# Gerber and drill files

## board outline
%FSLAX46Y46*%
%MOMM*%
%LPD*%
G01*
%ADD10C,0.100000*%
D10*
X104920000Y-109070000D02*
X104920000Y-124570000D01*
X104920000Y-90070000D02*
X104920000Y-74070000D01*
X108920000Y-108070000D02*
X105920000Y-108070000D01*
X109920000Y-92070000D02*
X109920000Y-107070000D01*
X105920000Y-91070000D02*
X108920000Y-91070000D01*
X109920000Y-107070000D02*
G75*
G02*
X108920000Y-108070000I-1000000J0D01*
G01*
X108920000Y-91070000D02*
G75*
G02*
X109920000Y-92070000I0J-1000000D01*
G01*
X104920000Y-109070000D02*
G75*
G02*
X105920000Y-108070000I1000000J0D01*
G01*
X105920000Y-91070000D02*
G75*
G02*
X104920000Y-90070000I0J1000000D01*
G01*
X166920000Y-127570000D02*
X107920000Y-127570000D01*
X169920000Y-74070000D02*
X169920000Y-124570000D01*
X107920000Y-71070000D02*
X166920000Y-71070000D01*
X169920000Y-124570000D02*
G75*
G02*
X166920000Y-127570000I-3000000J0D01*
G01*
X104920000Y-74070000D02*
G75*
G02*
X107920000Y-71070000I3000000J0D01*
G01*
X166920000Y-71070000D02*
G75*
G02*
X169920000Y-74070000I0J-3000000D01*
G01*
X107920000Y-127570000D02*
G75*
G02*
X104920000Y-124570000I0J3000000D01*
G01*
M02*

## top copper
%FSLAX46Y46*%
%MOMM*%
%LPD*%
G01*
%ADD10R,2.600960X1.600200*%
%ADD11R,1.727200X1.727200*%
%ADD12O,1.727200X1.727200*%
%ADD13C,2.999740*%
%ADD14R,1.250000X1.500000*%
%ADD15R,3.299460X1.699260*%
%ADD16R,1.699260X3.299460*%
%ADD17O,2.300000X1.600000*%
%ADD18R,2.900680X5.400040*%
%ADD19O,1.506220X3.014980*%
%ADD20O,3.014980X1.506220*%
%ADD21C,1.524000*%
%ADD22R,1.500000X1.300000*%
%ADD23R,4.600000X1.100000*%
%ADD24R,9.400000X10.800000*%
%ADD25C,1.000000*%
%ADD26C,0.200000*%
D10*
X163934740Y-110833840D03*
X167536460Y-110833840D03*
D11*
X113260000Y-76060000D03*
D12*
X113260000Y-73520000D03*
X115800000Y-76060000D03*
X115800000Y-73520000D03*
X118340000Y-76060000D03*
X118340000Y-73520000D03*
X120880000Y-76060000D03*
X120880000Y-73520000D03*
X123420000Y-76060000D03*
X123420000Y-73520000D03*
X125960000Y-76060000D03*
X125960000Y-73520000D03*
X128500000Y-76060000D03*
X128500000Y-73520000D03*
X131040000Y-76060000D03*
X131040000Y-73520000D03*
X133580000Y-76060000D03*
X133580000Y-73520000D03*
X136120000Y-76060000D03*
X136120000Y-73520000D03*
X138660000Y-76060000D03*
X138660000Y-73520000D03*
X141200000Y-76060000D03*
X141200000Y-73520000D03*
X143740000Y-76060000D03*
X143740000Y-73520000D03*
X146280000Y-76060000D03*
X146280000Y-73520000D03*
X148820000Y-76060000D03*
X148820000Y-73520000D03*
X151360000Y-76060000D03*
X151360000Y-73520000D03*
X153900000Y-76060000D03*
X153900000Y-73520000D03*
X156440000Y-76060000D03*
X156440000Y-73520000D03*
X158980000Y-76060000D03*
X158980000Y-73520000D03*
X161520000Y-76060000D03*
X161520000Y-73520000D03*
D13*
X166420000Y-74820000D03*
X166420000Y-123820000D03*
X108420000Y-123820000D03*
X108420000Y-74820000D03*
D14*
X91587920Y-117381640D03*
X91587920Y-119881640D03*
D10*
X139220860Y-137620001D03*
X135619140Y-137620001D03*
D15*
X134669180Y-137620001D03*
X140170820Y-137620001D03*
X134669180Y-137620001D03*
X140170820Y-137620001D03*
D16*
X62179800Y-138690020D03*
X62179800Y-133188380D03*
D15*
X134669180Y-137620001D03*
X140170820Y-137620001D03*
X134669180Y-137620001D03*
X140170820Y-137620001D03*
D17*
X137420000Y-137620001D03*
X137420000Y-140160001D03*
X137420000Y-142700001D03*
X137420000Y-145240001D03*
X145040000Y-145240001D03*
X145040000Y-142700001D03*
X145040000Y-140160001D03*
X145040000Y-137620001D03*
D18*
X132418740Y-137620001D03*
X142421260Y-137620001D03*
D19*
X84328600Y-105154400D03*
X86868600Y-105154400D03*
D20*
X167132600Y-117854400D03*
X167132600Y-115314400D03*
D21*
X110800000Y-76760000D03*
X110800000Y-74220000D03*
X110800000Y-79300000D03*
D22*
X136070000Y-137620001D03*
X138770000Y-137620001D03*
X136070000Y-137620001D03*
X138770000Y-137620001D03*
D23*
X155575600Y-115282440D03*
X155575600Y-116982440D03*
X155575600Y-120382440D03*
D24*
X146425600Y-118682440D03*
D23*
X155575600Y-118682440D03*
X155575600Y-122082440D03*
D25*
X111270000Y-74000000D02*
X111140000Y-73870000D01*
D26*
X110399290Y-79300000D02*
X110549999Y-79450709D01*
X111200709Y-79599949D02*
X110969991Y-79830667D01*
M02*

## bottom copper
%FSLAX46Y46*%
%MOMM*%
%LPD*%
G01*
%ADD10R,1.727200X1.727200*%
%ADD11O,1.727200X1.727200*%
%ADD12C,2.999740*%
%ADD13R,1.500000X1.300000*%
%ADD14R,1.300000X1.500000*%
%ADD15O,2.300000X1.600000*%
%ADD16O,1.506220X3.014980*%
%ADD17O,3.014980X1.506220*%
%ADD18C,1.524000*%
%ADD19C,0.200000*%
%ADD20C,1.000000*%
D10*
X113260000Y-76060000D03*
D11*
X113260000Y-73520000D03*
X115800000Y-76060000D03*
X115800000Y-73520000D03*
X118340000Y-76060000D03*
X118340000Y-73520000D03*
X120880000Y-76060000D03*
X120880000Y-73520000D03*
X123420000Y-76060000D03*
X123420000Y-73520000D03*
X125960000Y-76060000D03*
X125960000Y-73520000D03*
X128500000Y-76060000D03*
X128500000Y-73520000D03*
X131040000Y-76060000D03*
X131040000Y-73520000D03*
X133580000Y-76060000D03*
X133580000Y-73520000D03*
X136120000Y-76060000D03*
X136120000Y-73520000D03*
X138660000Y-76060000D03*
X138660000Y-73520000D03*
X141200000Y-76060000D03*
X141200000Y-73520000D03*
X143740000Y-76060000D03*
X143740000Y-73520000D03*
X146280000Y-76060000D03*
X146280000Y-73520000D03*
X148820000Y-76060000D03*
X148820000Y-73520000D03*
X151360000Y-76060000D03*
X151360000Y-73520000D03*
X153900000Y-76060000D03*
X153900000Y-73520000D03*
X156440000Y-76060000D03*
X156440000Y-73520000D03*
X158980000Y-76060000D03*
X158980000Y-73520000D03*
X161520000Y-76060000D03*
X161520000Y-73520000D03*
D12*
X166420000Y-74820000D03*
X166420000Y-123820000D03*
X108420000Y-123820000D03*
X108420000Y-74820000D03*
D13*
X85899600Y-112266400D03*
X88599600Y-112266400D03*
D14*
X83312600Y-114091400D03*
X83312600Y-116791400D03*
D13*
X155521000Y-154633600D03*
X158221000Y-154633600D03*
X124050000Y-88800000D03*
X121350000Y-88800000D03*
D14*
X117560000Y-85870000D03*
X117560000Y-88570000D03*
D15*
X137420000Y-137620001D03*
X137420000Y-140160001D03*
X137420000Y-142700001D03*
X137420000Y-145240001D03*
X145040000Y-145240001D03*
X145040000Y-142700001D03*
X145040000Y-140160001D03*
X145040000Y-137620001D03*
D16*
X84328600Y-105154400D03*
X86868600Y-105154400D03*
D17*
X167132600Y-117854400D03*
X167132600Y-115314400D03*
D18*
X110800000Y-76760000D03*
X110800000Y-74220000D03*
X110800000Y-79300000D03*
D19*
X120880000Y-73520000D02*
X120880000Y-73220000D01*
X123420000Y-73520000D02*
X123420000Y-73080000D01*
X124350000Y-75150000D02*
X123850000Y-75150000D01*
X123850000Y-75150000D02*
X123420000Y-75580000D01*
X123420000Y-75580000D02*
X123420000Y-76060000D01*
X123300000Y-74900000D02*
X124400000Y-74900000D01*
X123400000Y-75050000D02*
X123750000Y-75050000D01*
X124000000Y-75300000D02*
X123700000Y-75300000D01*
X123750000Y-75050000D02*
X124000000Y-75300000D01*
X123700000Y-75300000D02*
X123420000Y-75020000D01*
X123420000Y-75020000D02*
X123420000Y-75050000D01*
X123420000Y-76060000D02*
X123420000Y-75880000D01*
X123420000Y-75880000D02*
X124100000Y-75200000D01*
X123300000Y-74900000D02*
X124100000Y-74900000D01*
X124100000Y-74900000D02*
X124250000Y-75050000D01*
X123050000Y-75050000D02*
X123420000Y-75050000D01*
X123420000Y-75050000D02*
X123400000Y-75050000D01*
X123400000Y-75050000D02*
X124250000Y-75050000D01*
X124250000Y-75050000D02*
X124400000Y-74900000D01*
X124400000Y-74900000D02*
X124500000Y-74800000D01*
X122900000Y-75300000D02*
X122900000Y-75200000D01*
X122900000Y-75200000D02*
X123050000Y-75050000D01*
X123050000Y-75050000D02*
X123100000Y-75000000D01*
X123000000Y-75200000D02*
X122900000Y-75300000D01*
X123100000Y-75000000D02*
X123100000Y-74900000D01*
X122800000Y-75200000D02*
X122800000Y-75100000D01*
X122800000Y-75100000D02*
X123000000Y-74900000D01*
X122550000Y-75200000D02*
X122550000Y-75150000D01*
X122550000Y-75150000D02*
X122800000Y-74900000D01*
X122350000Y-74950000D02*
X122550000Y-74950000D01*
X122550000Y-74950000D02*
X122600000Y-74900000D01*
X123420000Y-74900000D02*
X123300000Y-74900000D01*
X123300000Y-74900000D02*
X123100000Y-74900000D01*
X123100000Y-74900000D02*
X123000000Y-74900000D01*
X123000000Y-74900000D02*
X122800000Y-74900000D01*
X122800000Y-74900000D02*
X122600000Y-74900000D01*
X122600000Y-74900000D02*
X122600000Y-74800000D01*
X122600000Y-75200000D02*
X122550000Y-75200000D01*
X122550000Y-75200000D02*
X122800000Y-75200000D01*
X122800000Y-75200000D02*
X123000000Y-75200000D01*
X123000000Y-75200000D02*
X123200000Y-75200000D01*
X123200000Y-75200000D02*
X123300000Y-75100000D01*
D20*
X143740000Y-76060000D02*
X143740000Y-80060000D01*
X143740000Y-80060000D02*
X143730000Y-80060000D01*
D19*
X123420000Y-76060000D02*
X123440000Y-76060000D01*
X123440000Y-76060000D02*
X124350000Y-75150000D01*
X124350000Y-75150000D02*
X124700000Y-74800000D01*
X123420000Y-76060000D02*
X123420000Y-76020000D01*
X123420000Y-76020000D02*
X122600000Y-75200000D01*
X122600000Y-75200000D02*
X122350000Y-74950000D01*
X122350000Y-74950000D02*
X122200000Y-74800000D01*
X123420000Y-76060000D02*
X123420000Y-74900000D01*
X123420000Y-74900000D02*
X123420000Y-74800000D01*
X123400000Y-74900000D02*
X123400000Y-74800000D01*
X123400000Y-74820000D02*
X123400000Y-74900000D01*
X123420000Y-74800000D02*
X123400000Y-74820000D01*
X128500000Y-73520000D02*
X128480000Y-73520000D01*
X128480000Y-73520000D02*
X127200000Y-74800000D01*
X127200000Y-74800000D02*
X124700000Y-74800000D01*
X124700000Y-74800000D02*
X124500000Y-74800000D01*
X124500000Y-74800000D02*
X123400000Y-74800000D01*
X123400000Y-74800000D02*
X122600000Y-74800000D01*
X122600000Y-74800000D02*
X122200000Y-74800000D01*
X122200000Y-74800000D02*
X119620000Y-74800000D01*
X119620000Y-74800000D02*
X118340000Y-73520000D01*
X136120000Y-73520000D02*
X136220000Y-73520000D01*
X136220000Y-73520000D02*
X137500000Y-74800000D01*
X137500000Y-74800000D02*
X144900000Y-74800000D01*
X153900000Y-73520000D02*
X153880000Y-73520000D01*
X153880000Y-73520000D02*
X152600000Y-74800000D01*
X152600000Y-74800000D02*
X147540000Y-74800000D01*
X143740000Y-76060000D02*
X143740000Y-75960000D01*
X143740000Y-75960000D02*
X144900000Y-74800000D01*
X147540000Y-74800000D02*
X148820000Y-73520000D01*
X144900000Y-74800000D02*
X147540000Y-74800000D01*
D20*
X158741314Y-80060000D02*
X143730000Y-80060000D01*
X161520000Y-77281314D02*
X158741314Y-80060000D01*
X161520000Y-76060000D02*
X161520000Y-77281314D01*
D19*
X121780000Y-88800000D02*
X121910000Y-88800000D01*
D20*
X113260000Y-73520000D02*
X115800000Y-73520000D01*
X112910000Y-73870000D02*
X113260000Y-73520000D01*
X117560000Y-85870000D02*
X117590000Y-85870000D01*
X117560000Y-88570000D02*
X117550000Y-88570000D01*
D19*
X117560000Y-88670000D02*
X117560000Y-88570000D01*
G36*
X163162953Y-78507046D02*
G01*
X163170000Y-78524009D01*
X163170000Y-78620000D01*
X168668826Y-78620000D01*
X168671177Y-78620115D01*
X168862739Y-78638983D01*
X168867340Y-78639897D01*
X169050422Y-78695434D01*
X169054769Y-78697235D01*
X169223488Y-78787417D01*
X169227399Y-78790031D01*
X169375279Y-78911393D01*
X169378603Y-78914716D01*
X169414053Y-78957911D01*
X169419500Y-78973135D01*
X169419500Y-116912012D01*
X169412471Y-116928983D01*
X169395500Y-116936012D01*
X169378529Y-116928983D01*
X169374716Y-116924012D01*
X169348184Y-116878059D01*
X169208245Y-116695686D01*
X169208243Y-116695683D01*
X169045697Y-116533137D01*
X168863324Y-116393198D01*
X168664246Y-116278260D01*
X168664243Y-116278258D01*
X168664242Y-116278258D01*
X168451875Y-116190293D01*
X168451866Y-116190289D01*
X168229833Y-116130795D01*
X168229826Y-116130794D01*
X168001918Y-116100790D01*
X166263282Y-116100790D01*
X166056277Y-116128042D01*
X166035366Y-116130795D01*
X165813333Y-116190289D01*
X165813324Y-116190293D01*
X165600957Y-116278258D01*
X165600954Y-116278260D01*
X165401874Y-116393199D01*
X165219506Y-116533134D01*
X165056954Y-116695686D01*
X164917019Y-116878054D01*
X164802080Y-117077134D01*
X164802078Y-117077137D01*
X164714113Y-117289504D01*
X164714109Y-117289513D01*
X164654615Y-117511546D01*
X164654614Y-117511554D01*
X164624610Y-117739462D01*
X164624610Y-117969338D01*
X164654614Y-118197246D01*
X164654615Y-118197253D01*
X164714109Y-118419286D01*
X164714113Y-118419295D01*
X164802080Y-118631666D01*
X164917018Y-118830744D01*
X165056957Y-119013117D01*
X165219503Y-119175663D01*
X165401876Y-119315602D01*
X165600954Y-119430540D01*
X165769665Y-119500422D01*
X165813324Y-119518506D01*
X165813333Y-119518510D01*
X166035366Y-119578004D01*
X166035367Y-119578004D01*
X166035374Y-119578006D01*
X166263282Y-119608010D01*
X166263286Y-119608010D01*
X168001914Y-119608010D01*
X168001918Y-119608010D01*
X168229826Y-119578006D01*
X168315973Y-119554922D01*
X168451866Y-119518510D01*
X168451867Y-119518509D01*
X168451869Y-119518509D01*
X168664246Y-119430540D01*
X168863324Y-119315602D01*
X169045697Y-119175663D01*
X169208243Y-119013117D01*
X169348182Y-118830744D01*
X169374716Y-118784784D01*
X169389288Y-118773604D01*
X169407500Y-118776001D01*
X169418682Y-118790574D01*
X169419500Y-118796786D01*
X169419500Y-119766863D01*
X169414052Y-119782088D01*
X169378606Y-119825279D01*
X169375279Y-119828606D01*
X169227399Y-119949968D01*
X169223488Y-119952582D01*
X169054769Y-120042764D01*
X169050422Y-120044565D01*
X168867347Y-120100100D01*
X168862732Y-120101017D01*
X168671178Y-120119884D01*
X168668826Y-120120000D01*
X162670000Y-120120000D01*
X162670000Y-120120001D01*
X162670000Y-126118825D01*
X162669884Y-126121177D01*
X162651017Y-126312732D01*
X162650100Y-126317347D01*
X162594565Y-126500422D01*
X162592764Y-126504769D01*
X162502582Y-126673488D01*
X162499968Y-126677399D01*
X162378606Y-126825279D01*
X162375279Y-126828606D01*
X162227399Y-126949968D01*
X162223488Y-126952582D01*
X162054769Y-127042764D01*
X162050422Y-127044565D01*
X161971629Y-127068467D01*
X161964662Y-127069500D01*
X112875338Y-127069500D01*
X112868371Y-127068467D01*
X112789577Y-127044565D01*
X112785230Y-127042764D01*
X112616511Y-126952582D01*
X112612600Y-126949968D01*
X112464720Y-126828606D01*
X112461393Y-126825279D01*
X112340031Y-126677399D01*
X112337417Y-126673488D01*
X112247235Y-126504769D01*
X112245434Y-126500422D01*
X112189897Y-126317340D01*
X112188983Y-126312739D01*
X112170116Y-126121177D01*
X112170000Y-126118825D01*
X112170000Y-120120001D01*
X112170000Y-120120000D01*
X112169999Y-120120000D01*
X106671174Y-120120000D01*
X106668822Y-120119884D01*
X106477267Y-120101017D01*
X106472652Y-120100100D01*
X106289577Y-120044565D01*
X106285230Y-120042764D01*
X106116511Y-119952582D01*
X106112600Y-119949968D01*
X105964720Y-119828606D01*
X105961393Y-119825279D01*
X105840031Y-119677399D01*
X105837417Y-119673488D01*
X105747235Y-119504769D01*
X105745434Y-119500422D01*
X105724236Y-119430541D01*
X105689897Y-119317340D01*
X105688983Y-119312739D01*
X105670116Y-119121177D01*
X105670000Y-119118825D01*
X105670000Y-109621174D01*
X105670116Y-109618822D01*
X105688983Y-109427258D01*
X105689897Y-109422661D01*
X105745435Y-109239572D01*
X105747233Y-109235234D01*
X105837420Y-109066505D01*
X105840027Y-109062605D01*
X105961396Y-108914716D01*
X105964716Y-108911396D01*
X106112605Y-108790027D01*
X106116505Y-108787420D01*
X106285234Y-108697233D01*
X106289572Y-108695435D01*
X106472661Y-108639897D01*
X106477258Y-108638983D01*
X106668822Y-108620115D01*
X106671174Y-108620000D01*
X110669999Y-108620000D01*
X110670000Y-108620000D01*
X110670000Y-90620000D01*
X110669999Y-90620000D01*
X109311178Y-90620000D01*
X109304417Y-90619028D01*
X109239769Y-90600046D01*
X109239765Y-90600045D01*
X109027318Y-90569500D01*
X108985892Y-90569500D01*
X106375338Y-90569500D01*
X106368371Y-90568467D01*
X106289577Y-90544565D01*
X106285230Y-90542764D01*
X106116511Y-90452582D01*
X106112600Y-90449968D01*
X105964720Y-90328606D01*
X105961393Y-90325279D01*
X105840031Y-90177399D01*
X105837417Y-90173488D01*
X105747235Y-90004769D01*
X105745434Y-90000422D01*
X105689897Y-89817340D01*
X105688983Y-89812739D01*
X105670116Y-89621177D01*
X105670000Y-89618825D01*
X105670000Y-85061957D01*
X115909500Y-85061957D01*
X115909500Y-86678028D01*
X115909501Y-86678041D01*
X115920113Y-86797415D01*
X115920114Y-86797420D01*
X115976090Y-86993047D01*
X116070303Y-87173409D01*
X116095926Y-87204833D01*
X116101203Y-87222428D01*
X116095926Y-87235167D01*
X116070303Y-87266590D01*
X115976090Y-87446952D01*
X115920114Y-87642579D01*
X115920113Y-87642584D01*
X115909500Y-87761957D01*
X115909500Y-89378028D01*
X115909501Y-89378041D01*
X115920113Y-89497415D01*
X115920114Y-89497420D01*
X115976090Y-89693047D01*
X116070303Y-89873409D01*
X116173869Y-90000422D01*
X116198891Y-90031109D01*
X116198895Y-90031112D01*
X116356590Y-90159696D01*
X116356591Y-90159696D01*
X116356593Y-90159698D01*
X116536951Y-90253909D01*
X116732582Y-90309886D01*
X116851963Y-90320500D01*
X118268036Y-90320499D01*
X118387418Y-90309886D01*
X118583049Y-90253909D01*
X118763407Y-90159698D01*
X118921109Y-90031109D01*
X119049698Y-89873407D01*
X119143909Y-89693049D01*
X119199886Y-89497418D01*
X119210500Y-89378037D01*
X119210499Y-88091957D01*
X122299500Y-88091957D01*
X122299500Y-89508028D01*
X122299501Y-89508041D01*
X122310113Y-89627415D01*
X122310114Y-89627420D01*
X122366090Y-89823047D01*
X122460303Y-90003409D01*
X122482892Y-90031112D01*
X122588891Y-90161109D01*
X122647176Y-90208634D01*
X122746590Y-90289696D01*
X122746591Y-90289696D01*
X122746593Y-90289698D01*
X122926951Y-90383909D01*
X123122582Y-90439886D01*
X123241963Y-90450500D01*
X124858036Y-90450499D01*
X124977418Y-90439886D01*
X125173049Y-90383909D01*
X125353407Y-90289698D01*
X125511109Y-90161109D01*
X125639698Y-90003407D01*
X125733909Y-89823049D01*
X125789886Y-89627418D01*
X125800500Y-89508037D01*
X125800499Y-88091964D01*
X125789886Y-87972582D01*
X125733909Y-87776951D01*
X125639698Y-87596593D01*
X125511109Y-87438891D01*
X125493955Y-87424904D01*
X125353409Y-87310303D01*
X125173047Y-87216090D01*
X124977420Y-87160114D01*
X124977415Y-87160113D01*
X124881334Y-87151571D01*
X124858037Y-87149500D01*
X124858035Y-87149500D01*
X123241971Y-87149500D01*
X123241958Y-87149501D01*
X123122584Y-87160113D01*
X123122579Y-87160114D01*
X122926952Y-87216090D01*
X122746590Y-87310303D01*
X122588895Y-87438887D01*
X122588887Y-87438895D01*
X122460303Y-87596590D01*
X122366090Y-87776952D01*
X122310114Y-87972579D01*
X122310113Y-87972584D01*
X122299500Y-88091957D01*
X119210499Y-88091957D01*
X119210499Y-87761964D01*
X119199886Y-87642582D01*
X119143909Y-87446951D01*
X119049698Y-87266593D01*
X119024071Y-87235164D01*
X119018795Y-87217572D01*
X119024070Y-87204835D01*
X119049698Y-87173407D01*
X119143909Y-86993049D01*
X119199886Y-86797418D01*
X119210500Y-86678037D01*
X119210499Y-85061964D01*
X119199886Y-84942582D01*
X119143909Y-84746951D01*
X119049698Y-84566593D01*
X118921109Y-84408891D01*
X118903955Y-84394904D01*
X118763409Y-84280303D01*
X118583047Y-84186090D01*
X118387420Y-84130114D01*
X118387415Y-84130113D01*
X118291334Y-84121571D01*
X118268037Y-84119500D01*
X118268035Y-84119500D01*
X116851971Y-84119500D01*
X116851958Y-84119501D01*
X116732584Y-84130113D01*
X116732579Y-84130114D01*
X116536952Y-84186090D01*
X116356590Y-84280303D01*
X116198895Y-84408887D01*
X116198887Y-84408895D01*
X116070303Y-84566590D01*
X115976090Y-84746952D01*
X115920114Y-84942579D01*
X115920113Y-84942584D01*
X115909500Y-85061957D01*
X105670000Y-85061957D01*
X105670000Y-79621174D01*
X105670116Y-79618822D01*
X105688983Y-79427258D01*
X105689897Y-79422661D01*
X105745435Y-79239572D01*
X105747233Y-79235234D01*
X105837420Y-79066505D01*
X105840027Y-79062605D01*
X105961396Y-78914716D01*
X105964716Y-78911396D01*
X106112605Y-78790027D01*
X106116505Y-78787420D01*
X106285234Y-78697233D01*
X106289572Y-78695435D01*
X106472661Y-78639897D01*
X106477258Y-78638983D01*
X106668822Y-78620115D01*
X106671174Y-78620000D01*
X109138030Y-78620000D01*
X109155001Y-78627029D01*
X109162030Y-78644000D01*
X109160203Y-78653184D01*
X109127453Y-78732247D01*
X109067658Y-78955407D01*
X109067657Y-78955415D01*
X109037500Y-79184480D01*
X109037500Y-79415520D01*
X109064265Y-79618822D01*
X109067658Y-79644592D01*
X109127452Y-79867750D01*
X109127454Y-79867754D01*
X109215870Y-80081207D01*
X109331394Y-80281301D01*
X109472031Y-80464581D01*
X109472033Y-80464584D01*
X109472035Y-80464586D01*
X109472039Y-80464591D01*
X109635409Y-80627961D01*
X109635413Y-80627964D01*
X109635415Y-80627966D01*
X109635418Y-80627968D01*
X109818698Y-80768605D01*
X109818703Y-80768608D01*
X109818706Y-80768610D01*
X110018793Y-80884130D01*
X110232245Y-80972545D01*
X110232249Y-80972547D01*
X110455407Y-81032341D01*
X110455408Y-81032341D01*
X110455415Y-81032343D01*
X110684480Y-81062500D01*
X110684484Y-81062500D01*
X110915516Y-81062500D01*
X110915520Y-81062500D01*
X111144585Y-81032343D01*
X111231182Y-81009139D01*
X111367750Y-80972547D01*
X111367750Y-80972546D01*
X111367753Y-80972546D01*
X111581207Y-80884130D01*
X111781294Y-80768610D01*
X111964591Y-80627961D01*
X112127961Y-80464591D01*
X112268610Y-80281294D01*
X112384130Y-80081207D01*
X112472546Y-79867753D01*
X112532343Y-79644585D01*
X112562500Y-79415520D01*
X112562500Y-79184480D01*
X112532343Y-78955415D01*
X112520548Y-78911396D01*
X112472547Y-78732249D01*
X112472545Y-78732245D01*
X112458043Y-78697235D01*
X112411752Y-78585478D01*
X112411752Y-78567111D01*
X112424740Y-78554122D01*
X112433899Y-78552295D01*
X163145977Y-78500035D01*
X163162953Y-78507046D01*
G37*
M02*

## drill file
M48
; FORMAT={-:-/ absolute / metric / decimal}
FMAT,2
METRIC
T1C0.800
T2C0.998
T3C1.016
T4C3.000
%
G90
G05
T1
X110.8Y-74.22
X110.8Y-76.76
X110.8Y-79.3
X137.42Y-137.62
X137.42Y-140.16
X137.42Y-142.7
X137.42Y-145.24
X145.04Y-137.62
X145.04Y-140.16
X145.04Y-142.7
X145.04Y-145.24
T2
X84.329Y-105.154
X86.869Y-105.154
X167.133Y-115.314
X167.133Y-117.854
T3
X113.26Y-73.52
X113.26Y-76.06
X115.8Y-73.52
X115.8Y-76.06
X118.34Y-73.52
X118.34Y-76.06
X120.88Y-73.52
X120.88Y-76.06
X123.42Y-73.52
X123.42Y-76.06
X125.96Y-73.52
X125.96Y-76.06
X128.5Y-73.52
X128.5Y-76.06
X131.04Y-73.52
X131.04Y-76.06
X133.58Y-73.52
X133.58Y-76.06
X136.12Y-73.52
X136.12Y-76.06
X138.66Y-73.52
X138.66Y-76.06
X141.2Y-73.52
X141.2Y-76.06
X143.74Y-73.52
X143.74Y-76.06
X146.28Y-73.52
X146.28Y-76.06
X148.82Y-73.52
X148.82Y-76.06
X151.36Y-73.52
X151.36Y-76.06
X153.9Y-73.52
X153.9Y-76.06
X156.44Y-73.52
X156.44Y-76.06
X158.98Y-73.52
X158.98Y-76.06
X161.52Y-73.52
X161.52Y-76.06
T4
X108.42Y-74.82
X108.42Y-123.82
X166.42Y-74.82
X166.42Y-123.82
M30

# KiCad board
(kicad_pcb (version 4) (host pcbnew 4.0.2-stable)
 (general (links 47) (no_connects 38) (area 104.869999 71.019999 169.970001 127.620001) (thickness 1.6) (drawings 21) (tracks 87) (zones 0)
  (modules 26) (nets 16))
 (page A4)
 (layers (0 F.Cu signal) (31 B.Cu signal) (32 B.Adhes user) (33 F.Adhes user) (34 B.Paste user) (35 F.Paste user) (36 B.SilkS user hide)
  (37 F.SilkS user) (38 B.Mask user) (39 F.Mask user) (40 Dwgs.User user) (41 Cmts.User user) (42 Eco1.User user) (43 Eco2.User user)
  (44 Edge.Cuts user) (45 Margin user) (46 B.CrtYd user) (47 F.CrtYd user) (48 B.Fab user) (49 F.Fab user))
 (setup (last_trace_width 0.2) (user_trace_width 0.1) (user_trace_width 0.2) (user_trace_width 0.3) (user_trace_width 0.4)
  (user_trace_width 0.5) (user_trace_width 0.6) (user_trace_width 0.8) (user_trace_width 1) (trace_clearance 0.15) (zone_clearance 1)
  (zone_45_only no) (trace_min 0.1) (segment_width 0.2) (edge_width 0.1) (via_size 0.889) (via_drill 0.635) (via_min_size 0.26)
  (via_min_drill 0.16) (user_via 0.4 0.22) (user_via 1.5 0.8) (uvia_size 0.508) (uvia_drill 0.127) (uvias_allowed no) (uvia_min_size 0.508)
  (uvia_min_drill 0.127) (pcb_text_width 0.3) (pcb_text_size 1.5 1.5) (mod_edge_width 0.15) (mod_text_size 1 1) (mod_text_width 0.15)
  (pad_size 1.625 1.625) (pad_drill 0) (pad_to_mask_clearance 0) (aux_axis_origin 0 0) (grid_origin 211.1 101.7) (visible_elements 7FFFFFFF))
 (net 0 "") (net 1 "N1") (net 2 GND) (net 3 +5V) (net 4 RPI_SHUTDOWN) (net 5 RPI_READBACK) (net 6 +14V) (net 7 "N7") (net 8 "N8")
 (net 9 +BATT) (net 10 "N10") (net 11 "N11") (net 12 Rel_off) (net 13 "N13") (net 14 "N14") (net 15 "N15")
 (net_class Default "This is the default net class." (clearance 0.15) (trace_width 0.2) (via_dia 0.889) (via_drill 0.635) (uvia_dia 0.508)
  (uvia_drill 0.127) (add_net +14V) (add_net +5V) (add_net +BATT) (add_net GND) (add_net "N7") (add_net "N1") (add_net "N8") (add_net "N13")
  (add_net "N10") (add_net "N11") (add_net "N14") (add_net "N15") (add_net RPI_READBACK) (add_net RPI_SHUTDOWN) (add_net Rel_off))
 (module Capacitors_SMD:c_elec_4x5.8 (layer F.Cu) (at 165.7356 110.83384 180)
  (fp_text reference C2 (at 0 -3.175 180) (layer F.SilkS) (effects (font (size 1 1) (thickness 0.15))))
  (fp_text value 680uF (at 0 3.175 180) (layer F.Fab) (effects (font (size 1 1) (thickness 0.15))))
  (pad 1 smd rect (at 1.80086 0 180) (size 2.60096 1.6002) (layers F.Cu F.Paste F.Mask) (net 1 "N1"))
  (pad 2 smd rect (at -1.80086 0 180) (size 2.60096 1.6002) (layers F.Cu F.Paste F.Mask) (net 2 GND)))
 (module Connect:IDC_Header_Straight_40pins (layer F.Cu) (at 113.26 76.06)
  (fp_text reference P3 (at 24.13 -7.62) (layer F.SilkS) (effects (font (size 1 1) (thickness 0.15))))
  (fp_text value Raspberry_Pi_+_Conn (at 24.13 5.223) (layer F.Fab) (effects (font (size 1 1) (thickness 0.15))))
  (pad 1 thru_hole rect (at 0 0) (size 1.7272 1.7272) (drill 1.016) (layers *.Cu *.Mask F.SilkS))
  (pad 2 thru_hole oval (at 0 -2.54) (size 1.7272 1.7272) (drill 1.016) (layers *.Cu *.Mask F.SilkS) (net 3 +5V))
  (pad 3 thru_hole oval (at 2.54 0) (size 1.7272 1.7272) (drill 1.016) (layers *.Cu *.Mask F.SilkS))
  (pad 4 thru_hole oval (at 2.54 -2.54) (size 1.7272 1.7272) (drill 1.016) (layers *.Cu *.Mask F.SilkS) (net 3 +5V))
  (pad 5 thru_hole oval (at 5.08 0) (size 1.7272 1.7272) (drill 1.016) (layers *.Cu *.Mask F.SilkS))
  (pad 6 thru_hole oval (at 5.08 -2.54) (size 1.7272 1.7272) (drill 1.016) (layers *.Cu *.Mask F.SilkS) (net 2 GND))
  (pad 7 thru_hole oval (at 7.62 0) (size 1.7272 1.7272) (drill 1.016) (layers *.Cu *.Mask F.SilkS))
  (pad 8 thru_hole oval (at 7.62 -2.54) (size 1.7272 1.7272) (drill 1.016) (layers *.Cu *.Mask F.SilkS))
  (pad 9 thru_hole oval (at 10.16 0) (size 1.7272 1.7272) (drill 1.016) (layers *.Cu *.Mask F.SilkS) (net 2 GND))
  (pad 10 thru_hole oval (at 10.16 -2.54) (size 1.7272 1.7272) (drill 1.016) (layers *.Cu *.Mask F.SilkS))
  (pad 11 thru_hole oval (at 12.7 0) (size 1.7272 1.7272) (drill 1.016) (layers *.Cu *.Mask F.SilkS))
  (pad 12 thru_hole oval (at 12.7 -2.54) (size 1.7272 1.7272) (drill 1.016) (layers *.Cu *.Mask F.SilkS))
  (pad 13 thru_hole oval (at 15.24 0) (size 1.7272 1.7272) (drill 1.016) (layers *.Cu *.Mask F.SilkS))
  (pad 14 thru_hole oval (at 15.24 -2.54) (size 1.7272 1.7272) (drill 1.016) (layers *.Cu *.Mask F.SilkS) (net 2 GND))
  (pad 15 thru_hole oval (at 17.78 0) (size 1.7272 1.7272) (drill 1.016) (layers *.Cu *.Mask F.SilkS))
  (pad 16 thru_hole oval (at 17.78 -2.54) (size 1.7272 1.7272) (drill 1.016) (layers *.Cu *.Mask F.SilkS))
  (pad 17 thru_hole oval (at 20.32 0) (size 1.7272 1.7272) (drill 1.016) (layers *.Cu *.Mask F.SilkS))
  (pad 18 thru_hole oval (at 20.32 -2.54) (size 1.7272 1.7272) (drill 1.016) (layers *.Cu *.Mask F.SilkS))
  (pad 19 thru_hole oval (at 22.86 0) (size 1.7272 1.7272) (drill 1.016) (layers *.Cu *.Mask F.SilkS))
  (pad 20 thru_hole oval (at 22.86 -2.54) (size 1.7272 1.7272) (drill 1.016) (layers *.Cu *.Mask F.SilkS) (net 2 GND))
  (pad 21 thru_hole oval (at 25.4 0) (size 1.7272 1.7272) (drill 1.016) (layers *.Cu *.Mask F.SilkS))
  (pad 22 thru_hole oval (at 25.4 -2.54) (size 1.7272 1.7272) (drill 1.016) (layers *.Cu *.Mask F.SilkS))
  (pad 23 thru_hole oval (at 27.94 0) (size 1.7272 1.7272) (drill 1.016) (layers *.Cu *.Mask F.SilkS))
  (pad 24 thru_hole oval (at 27.94 -2.54) (size 1.7272 1.7272) (drill 1.016) (layers *.Cu *.Mask F.SilkS))
  (pad 25 thru_hole oval (at 30.48 0) (size 1.7272 1.7272) (drill 1.016) (layers *.Cu *.Mask F.SilkS) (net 2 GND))
  (pad 26 thru_hole oval (at 30.48 -2.54) (size 1.7272 1.7272) (drill 1.016) (layers *.Cu *.Mask F.SilkS))
  (pad 27 thru_hole oval (at 33.02 0) (size 1.7272 1.7272) (drill 1.016) (layers *.Cu *.Mask F.SilkS))
  (pad 28 thru_hole oval (at 33.02 -2.54) (size 1.7272 1.7272) (drill 1.016) (layers *.Cu *.Mask F.SilkS))
  (pad 29 thru_hole oval (at 35.56 0) (size 1.7272 1.7272) (drill 1.016) (layers *.Cu *.Mask F.SilkS) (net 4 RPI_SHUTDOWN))
  (pad 30 thru_hole oval (at 35.56 -2.54) (size 1.7272 1.7272) (drill 1.016) (layers *.Cu *.Mask F.SilkS) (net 2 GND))
  (pad 31 thru_hole oval (at 38.1 0) (size 1.7272 1.7272) (drill 1.016) (layers *.Cu *.Mask F.SilkS) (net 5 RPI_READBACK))
  (pad 32 thru_hole oval (at 38.1 -2.54) (size 1.7272 1.7272) (drill 1.016) (layers *.Cu *.Mask F.SilkS))
  (pad 33 thru_hole oval (at 40.64 0) (size 1.7272 1.7272) (drill 1.016) (layers *.Cu *.Mask F.SilkS))
  (pad 34 thru_hole oval (at 40.64 -2.54) (size 1.7272 1.7272) (drill 1.016) (layers *.Cu *.Mask F.SilkS) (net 2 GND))
  (pad 35 thru_hole oval (at 43.18 0) (size 1.7272 1.7272) (drill 1.016) (layers *.Cu *.Mask F.SilkS))
  (pad 36 thru_hole oval (at 43.18 -2.54) (size 1.7272 1.7272) (drill 1.016) (layers *.Cu *.Mask F.SilkS))
  (pad 37 thru_hole oval (at 45.72 0) (size 1.7272 1.7272) (drill 1.016) (layers *.Cu *.Mask F.SilkS))
  (pad 38 thru_hole oval (at 45.72 -2.54) (size 1.7272 1.7272) (drill 1.016) (layers *.Cu *.Mask F.SilkS))
  (pad 39 thru_hole oval (at 48.26 0) (size 1.7272 1.7272) (drill 1.016) (layers *.Cu *.Mask F.SilkS) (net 2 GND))
  (pad 40 thru_hole oval (at 48.26 -2.54) (size 1.7272 1.7272) (drill 1.016) (layers *.Cu *.Mask F.SilkS)))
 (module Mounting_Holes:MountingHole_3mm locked (layer F.Cu) (at 166.42 74.82)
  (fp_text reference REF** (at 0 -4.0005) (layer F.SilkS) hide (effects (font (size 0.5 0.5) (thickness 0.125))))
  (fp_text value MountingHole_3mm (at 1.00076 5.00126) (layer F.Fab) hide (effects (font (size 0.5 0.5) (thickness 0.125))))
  (pad 1 thru_hole circle (at 0 0) (size 2.99974 2.99974) (drill 2.99974) (layers)))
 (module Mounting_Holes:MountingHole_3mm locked (layer F.Cu) (at 166.42 123.82)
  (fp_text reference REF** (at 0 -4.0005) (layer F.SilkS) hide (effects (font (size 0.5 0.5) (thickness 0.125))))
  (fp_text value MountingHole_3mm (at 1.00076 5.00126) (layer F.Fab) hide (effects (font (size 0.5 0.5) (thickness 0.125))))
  (pad 1 thru_hole circle (at 0 0) (size 2.99974 2.99974) (drill 2.99974) (layers)))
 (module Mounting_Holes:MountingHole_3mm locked (layer F.Cu) (at 108.42 123.82)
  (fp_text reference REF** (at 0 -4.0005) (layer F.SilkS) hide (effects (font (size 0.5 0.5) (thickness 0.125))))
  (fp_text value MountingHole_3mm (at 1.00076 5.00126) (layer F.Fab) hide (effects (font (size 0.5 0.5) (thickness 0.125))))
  (pad 1 thru_hole circle (at 0 0) (size 2.99974 2.99974) (drill 2.99974) (layers)))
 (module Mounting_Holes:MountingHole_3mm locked (layer F.Cu) (at 108.42 74.82)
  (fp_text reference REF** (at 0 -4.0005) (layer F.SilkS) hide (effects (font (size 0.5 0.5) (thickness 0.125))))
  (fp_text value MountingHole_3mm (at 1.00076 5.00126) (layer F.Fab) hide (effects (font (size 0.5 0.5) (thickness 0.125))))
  (pad 1 thru_hole circle (at 0 0) (size 2.99974 2.99974) (drill 2.99974) (layers)))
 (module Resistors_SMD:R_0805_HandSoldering (layer B.Cu) (at 87.2496 112.2664)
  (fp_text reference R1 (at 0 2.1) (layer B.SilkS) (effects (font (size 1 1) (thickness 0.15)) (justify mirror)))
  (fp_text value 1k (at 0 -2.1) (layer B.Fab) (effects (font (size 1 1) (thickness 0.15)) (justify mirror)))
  (pad 1 smd rect (at -1.35 0) (size 1.5 1.3) (layers B.Cu B.Paste B.Mask) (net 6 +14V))
  (pad 2 smd rect (at 1.35 0) (size 1.5 1.3) (layers B.Cu B.Paste B.Mask) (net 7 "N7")))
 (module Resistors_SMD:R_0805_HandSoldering (layer B.Cu) (at 83.3126 115.4414 270)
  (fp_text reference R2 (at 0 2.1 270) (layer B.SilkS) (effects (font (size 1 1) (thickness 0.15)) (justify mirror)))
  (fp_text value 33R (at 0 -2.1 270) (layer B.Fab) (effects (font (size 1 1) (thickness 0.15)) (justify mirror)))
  (pad 1 smd rect (at -1.35 0 270) (size 1.5 1.3) (layers B.Cu B.Paste B.Mask) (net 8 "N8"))
  (pad 2 smd rect (at 1.35 0 270) (size 1.5 1.3) (layers B.Cu B.Paste B.Mask) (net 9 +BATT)))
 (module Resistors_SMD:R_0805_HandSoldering (layer B.Cu) (at 156.871 154.6336)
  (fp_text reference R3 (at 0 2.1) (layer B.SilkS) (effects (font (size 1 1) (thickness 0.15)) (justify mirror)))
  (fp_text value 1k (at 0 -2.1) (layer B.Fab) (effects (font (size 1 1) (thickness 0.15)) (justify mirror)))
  (pad 1 smd rect (at -1.35 0) (size 1.5 1.3) (layers B.Cu B.Paste B.Mask))
  (pad 2 smd rect (at 1.35 0) (size 1.5 1.3) (layers B.Cu B.Paste B.Mask) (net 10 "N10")))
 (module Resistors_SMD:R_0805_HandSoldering (layer B.Cu) (at 122.7 88.8 180)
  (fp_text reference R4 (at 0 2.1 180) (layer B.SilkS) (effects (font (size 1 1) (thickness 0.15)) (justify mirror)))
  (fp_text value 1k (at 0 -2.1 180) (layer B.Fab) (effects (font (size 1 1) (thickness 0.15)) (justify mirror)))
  (pad 1 smd rect (at -1.35 0 180) (size 1.5 1.3) (layers B.Cu B.Paste B.Mask) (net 10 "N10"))
  (pad 2 smd rect (at 1.35 0 180) (size 1.5 1.3) (layers B.Cu B.Paste B.Mask) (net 2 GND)))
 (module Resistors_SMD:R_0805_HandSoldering (layer B.Cu) (at 117.56 87.22 270)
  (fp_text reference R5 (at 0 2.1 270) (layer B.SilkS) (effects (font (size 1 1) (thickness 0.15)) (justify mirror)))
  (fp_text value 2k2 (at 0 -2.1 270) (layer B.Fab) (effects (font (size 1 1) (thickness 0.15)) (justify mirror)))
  (pad 1 smd rect (at -1.35 0 270) (size 1.5 1.3) (layers B.Cu B.Paste B.Mask) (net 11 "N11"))
  (pad 2 smd rect (at 1.35 0 270) (size 1.5 1.3) (layers B.Cu B.Paste B.Mask) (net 4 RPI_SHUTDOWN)))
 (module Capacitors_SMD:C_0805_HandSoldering (layer F.Cu) (at 91.58792 118.63164 270)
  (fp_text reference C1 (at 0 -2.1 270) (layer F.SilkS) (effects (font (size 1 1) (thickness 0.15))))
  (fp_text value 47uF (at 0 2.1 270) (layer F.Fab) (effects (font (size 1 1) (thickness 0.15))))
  (pad 1 smd rect (at -1.25 0 270) (size 1.5 1.25) (layers F.Cu F.Paste F.Mask) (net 6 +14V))
  (pad 2 smd rect (at 1.25 0 270) (size 1.5 1.25) (layers F.Cu F.Paste F.Mask) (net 7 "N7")))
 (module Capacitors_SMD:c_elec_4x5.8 (layer F.Cu) (at 137.42 137.620001)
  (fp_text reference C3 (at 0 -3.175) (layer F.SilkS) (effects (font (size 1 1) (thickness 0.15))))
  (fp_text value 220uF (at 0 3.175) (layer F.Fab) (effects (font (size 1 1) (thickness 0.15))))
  (pad 1 smd rect (at 1.80086 0) (size 2.60096 1.6002) (layers F.Cu F.Paste F.Mask) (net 3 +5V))
  (pad 2 smd rect (at -1.80086 0) (size 2.60096 1.6002) (layers F.Cu F.Paste F.Mask) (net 2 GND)))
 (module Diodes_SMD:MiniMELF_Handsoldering (layer F.Cu) (at 137.42 137.620001)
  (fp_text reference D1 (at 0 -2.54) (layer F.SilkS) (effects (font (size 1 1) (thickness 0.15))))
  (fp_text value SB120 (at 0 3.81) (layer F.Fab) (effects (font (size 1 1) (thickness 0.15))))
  (pad 1 smd rect (at -2.75082 0) (size 3.29946 1.69926) (layers F.Cu F.Paste F.Mask) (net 3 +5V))
  (pad 2 smd rect (at 2.75082 0) (size 3.29946 1.69926) (layers F.Cu F.Paste F.Mask) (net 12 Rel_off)))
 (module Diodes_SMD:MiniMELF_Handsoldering (layer F.Cu) (at 137.42 137.620001)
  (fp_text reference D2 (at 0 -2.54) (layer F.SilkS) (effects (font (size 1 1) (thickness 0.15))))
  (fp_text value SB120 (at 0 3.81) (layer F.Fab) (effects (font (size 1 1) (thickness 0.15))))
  (pad 1 smd rect (at -2.75082 0) (size 3.29946 1.69926) (layers F.Cu F.Paste F.Mask) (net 8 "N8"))
  (pad 2 smd rect (at 2.75082 0) (size 3.29946 1.69926) (layers F.Cu F.Paste F.Mask) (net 6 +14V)))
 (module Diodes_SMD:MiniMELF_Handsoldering (layer F.Cu) (at 62.1798 135.9392 90)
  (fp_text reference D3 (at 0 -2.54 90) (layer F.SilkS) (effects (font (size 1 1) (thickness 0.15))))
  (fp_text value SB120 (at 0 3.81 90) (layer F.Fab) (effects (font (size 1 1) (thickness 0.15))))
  (pad 1 smd rect (at -2.75082 0 90) (size 3.29946 1.69926) (layers F.Cu F.Paste F.Mask) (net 8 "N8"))
  (pad 2 smd rect (at 2.75082 0 90) (size 3.29946 1.69926) (layers F.Cu F.Paste F.Mask) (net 9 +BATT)))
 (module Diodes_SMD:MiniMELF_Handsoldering (layer F.Cu) (at 137.42 137.620001)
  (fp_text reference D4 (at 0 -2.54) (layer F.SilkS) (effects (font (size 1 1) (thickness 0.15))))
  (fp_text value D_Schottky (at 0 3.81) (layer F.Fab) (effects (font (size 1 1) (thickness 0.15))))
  (pad 1 smd rect (at -2.75082 0) (size 3.29946 1.69926) (layers F.Cu F.Paste F.Mask) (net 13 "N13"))
  (pad 2 smd rect (at 2.75082 0) (size 3.29946 1.69926) (layers F.Cu F.Paste F.Mask) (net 2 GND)))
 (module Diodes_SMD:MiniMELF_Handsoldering (layer F.Cu) (at 137.42 137.620001)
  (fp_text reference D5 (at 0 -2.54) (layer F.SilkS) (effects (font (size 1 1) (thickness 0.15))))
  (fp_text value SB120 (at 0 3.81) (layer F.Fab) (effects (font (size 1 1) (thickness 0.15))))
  (pad 1 smd rect (at -2.75082 0) (size 3.29946 1.69926) (layers F.Cu F.Paste F.Mask) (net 3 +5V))
  (pad 2 smd rect (at 2.75082 0) (size 3.29946 1.69926) (layers F.Cu F.Paste F.Mask) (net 10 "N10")))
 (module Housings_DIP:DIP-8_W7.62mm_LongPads (layer F.Cu) (at 137.42 137.620001)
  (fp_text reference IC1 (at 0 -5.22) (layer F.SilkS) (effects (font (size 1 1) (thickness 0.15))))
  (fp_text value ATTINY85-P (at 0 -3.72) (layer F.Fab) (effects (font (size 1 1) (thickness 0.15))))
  (pad 1 thru_hole oval (at 0 0) (size 2.3 1.6) (drill 0.8) (layers *.Cu *.Mask F.SilkS))
  (pad 2 thru_hole oval (at 0 2.54) (size 2.3 1.6) (drill 0.8) (layers *.Cu *.Mask F.SilkS) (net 5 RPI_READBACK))
  (pad 3 thru_hole oval (at 0 5.08) (size 2.3 1.6) (drill 0.8) (layers *.Cu *.Mask F.SilkS))
  (pad 4 thru_hole oval (at 0 7.62) (size 2.3 1.6) (drill 0.8) (layers *.Cu *.Mask F.SilkS) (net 2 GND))
  (pad 5 thru_hole oval (at 7.62 7.62) (size 2.3 1.6) (drill 0.8) (layers *.Cu *.Mask F.SilkS) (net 10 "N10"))
  (pad 6 thru_hole oval (at 7.62 5.08) (size 2.3 1.6) (drill 0.8) (layers *.Cu *.Mask F.SilkS) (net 11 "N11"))
  (pad 7 thru_hole oval (at 7.62 2.54) (size 2.3 1.6) (drill 0.8) (layers *.Cu *.Mask F.SilkS) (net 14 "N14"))
  (pad 8 thru_hole oval (at 7.62 0) (size 2.3 1.6) (drill 0.8) (layers *.Cu *.Mask F.SilkS) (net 3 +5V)))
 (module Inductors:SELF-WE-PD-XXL (layer F.Cu) (at 137.42 137.620001)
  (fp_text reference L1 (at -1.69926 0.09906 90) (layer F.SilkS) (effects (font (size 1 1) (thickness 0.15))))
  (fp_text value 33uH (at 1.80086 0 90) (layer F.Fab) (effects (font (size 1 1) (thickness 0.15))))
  (pad 1 smd rect (at -5.00126 0) (size 2.90068 5.40004) (layers F.Cu F.Paste F.Mask) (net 3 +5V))
  (pad 2 smd rect (at 5.00126 0) (size 2.90068 5.40004) (layers F.Cu F.Paste F.Mask) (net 13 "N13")))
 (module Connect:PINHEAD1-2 (layer F.Cu) (at 85.5986 105.1544)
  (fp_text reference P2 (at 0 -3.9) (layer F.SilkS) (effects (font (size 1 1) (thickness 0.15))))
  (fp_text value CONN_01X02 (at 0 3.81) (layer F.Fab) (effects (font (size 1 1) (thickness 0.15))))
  (pad 1 thru_hole oval (at -1.27 0) (size 1.50622 3.01498) (drill 0.99822) (layers *.Cu *.Mask) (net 9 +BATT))
  (pad 2 thru_hole oval (at 1.27 0) (size 1.50622 3.01498) (drill 0.99822) (layers *.Cu *.Mask) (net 2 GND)))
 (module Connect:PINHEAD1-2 (layer F.Cu) (at 167.1326 116.5844 90)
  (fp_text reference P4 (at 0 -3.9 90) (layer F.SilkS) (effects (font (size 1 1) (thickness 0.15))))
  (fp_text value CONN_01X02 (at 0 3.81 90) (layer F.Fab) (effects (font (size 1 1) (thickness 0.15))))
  (pad 1 thru_hole oval (at -1.27 0 90) (size 1.50622 3.01498) (drill 0.99822) (layers *.Cu *.Mask) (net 6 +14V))
  (pad 2 thru_hole oval (at 1.27 0 90) (size 1.50622 3.01498) (drill 0.99822) (layers *.Cu *.Mask) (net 2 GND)))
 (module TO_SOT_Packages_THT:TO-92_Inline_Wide (layer F.Cu) (at 110.8 79.3 90)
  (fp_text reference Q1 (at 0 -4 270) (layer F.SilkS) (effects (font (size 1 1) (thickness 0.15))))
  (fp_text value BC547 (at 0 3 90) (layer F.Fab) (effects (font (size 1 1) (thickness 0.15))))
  (pad 2 thru_hole circle (at 2.54 0 180) (size 1.524 1.524) (drill 0.8) (layers *.Cu *.Mask F.SilkS) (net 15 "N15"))
  (pad 3 thru_hole circle (at 5.08 0 180) (size 1.524 1.524) (drill 0.8) (layers *.Cu *.Mask F.SilkS) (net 2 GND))
  (pad 1 thru_hole circle (at 0 0 180) (size 1.524 1.524) (drill 0.8) (layers *.Cu *.Mask F.SilkS) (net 12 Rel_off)))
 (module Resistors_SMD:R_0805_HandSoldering (layer F.Cu) (at 137.42 137.620001)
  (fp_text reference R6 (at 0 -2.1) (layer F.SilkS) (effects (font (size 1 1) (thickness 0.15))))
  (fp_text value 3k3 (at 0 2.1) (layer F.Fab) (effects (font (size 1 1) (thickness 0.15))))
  (pad 1 smd rect (at -1.35 0) (size 1.5 1.3) (layers F.Cu F.Paste F.Mask) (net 4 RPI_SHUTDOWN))
  (pad 2 smd rect (at 1.35 0) (size 1.5 1.3) (layers F.Cu F.Paste F.Mask) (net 2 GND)))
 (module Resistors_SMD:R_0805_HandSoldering (layer F.Cu) (at 137.42 137.620001)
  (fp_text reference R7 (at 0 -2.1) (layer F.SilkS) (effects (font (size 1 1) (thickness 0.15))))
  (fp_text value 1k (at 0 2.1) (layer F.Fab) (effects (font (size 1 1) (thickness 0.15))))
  (pad 1 smd rect (at -1.35 0) (size 1.5 1.3) (layers F.Cu F.Paste F.Mask) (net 14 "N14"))
  (pad 2 smd rect (at 1.35 0) (size 1.5 1.3) (layers F.Cu F.Paste F.Mask) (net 15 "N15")))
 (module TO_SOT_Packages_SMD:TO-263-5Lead (layer F.Cu) (at 155.5756 118.68244 180)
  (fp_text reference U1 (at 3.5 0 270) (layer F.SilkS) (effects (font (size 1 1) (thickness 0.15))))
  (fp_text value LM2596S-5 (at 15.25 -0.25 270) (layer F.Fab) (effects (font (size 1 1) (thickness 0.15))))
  (pad 5 smd rect (at 0 3.4 180) (size 4.6 1.1) (layers F.Cu F.Paste F.Mask) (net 2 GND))
  (pad 4 smd rect (at 0 1.7 180) (size 4.6 1.1) (layers F.Cu F.Paste F.Mask) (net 3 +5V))
  (pad 2 smd rect (at 0 -1.7 180) (size 4.6 1.1) (layers F.Cu F.Paste F.Mask) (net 13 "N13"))
  (pad 3 smd rect (at 9.15 0 180) (size 9.4 10.8) (layers F.Cu F.Paste F.Mask) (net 2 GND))
  (pad 3 smd rect (at 0 0 180) (size 4.6 1.1) (layers F.Cu F.Paste F.Mask) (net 2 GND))
  (pad 1 smd rect (at 0 -3.4 180) (size 4.6 1.1) (layers F.Cu F.Paste F.Mask) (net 1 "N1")))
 (gr_line (start 104.92 109.07) (end 104.92 124.57) (angle 90) (layer Edge.Cuts) (width 0.1))
 (gr_line (start 104.92 90.07) (end 104.92 74.07) (angle 90) (layer Edge.Cuts) (width 0.1))
 (gr_line (start 108.92 108.07) (end 105.92 108.07) (angle 90) (layer Edge.Cuts) (width 0.1))
 (gr_line (start 109.92 92.07) (end 109.92 107.07) (angle 90) (layer Edge.Cuts) (width 0.1))
 (gr_line (start 105.92 91.07) (end 108.92 91.07) (angle 90) (layer Edge.Cuts) (width 0.1))
 (gr_arc (start 108.92 107.07) (end 109.92 107.07) (angle 90) (layer Edge.Cuts) (width 0.1))
 (gr_arc (start 108.92 92.07) (end 108.92 91.07) (angle 90) (layer Edge.Cuts) (width 0.1))
 (gr_arc (start 105.92 109.07) (end 104.92 109.07) (angle 90) (layer Edge.Cuts) (width 0.1))
 (gr_arc (start 105.92 90.07) (end 105.92 91.07) (angle 90) (layer Edge.Cuts) (width 0.1))
 (gr_line (start 166.92 127.57) (end 107.92 127.57) (angle 90) (layer Edge.Cuts) (width 0.1))
 (gr_line (start 169.92 74.07) (end 169.92 124.57) (angle 90) (layer Edge.Cuts) (width 0.1))
 (gr_line (start 107.92 71.07) (end 166.92 71.07) (angle 90) (layer Edge.Cuts) (width 0.1))
 (gr_arc (start 166.92 124.57) (end 169.92 124.57) (angle 90) (layer Edge.Cuts) (width 0.1))
 (gr_arc (start 107.92 74.07) (end 104.92 74.07) (angle 90) (layer Edge.Cuts) (width 0.1))
 (gr_arc (start 166.92 74.07) (end 166.92 71.07) (angle 90) (layer Edge.Cuts) (width 0.1))
 (gr_arc (start 107.92 124.57) (end 107.92 127.57) (angle 90) (layer Edge.Cuts) (width 0.1))
 (segment (start 120.88 73.52) (end 120.88 73.22) (width 0.2) (layer B.Cu) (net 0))
 (segment (start 123.42 73.52) (end 123.42 73.08) (width 0.2) (layer B.Cu) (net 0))
 (segment (start 124.35 75.15) (end 123.85 75.15) (width 0.2) (layer B.Cu) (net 2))
 (segment (start 123.85 75.15) (end 123.42 75.58) (width 0.2) (layer B.Cu) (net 2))
 (segment (start 123.42 75.58) (end 123.42 76.06) (width 0.2) (layer B.Cu) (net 2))
 (segment (start 123.3 74.9) (end 124.4 74.9) (width 0.2) (layer B.Cu) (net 2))
 (segment (start 123.4 75.05) (end 123.75 75.05) (width 0.2) (layer B.Cu) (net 2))
 (segment (start 124 75.3) (end 123.7 75.3) (width 0.2) (layer B.Cu) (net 2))
 (segment (start 123.75 75.05) (end 124 75.3) (width 0.2) (layer B.Cu) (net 2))
 (segment (start 123.7 75.3) (end 123.42 75.02) (width 0.2) (layer B.Cu) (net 2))
 (segment (start 123.42 75.02) (end 123.42 75.05) (width 0.2) (layer B.Cu) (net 2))
 (segment (start 123.42 76.06) (end 123.42 75.88) (width 0.2) (layer B.Cu) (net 2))
 (segment (start 123.42 75.88) (end 124.1 75.2) (width 0.2) (layer B.Cu) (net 2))
 (segment (start 123.3 74.9) (end 124.1 74.9) (width 0.2) (layer B.Cu) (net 2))
 (segment (start 124.1 74.9) (end 124.25 75.05) (width 0.2) (layer B.Cu) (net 2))
 (segment (start 123.05 75.05) (end 123.42 75.05) (width 0.2) (layer B.Cu) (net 2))
 (segment (start 123.42 75.05) (end 123.4 75.05) (width 0.2) (layer B.Cu) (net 2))
 (segment (start 123.4 75.05) (end 124.25 75.05) (width 0.2) (layer B.Cu) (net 2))
 (segment (start 124.25 75.05) (end 124.4 74.9) (width 0.2) (layer B.Cu) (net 2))
 (segment (start 124.4 74.9) (end 124.5 74.8) (width 0.2) (layer B.Cu) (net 2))
 (segment (start 122.9 75.3) (end 122.9 75.2) (width 0.2) (layer B.Cu) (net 2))
 (segment (start 122.9 75.2) (end 123.05 75.05) (width 0.2) (layer B.Cu) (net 2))
 (segment (start 123.05 75.05) (end 123.1 75) (width 0.2) (layer B.Cu) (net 2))
 (segment (start 123 75.2) (end 122.9 75.3) (width 0.2) (layer B.Cu) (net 2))
 (segment (start 123.1 75) (end 123.1 74.9) (width 0.2) (layer B.Cu) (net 2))
 (segment (start 122.8 75.2) (end 122.8 75.1) (width 0.2) (layer B.Cu) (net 2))
 (segment (start 122.8 75.1) (end 123 74.9) (width 0.2) (layer B.Cu) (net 2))
 (segment (start 122.55 75.2) (end 122.55 75.15) (width 0.2) (layer B.Cu) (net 2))
 (segment (start 122.55 75.15) (end 122.8 74.9) (width 0.2) (layer B.Cu) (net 2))
 (segment (start 122.35 74.95) (end 122.55 74.95) (width 0.2) (layer B.Cu) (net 2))
 (segment (start 122.55 74.95) (end 122.6 74.9) (width 0.2) (layer B.Cu) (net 2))
 (segment (start 123.42 74.9) (end 123.3 74.9) (width 0.2) (layer B.Cu) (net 2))
 (segment (start 123.3 74.9) (end 123.1 74.9) (width 0.2) (layer B.Cu) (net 2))
 (segment (start 123.1 74.9) (end 123 74.9) (width 0.2) (layer B.Cu) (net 2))
 (segment (start 123 74.9) (end 122.8 74.9) (width 0.2) (layer B.Cu) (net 2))
 (segment (start 122.8 74.9) (end 122.6 74.9) (width 0.2) (layer B.Cu) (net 2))
 (segment (start 122.6 74.9) (end 122.6 74.8) (width 0.2) (layer B.Cu) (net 2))
 (segment (start 122.6 75.2) (end 122.55 75.2) (width 0.2) (layer B.Cu) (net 2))
 (segment (start 122.55 75.2) (end 122.8 75.2) (width 0.2) (layer B.Cu) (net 2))
 (segment (start 122.8 75.2) (end 123 75.2) (width 0.2) (layer B.Cu) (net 2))
 (segment (start 123 75.2) (end 123.2 75.2) (width 0.2) (layer B.Cu) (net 2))
 (segment (start 123.2 75.2) (end 123.3 75.1) (width 0.2) (layer B.Cu) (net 2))
 (segment (start 143.74 76.06) (end 143.74 80.06) (width 1) (layer B.Cu) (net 2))
 (segment (start 143.74 80.06) (end 143.73 80.06) (width 1) (layer B.Cu) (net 2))
 (segment (start 123.42 76.06) (end 123.44 76.06) (width 0.2) (layer B.Cu) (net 2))
 (segment (start 123.44 76.06) (end 124.35 75.15) (width 0.2) (layer B.Cu) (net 2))
 (segment (start 124.35 75.15) (end 124.7 74.8) (width 0.2) (layer B.Cu) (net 2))
 (segment (start 123.42 76.06) (end 123.42 76.02) (width 0.2) (layer B.Cu) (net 2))
 (segment (start 123.42 76.02) (end 122.6 75.2) (width 0.2) (layer B.Cu) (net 2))
 (segment (start 122.6 75.2) (end 122.35 74.95) (width 0.2) (layer B.Cu) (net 2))
 (segment (start 122.35 74.95) (end 122.2 74.8) (width 0.2) (layer B.Cu) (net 2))
 (segment (start 123.42 76.06) (end 123.42 74.9) (width 0.2) (layer B.Cu) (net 2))
 (segment (start 123.42 74.9) (end 123.42 74.8) (width 0.2) (layer B.Cu) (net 2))
 (segment (start 123.4 74.9) (end 123.4 74.8) (width 0.2) (layer B.Cu) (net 2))
 (segment (start 123.4 74.82) (end 123.4 74.9) (width 0.2) (layer B.Cu) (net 2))
 (segment (start 123.42 74.8) (end 123.4 74.82) (width 0.2) (layer B.Cu) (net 2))
 (segment (start 128.5 73.52) (end 128.48 73.52) (width 0.2) (layer B.Cu) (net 2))
 (segment (start 128.48 73.52) (end 127.2 74.8) (width 0.2) (layer B.Cu) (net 2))
 (segment (start 127.2 74.8) (end 124.7 74.8) (width 0.2) (layer B.Cu) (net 2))
 (segment (start 124.7 74.8) (end 124.5 74.8) (width 0.2) (layer B.Cu) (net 2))
 (segment (start 124.5 74.8) (end 123.4 74.8) (width 0.2) (layer B.Cu) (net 2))
 (segment (start 123.4 74.8) (end 122.6 74.8) (width 0.2) (layer B.Cu) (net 2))
 (segment (start 122.6 74.8) (end 122.2 74.8) (width 0.2) (layer B.Cu) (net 2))
 (segment (start 122.2 74.8) (end 119.62 74.8) (width 0.2) (layer B.Cu) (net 2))
 (segment (start 119.62 74.8) (end 118.34 73.52) (width 0.2) (layer B.Cu) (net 2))
 (segment (start 136.12 73.52) (end 136.22 73.52) (width 0.2) (layer B.Cu) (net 2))
 (segment (start 136.22 73.52) (end 137.5 74.8) (width 0.2) (layer B.Cu) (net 2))
 (segment (start 137.5 74.8) (end 144.9 74.8) (width 0.2) (layer B.Cu) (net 2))
 (segment (start 153.9 73.52) (end 153.88 73.52) (width 0.2) (layer B.Cu) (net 2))
 (segment (start 153.88 73.52) (end 152.6 74.8) (width 0.2) (layer B.Cu) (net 2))
 (segment (start 152.6 74.8) (end 147.54 74.8) (width 0.2) (layer B.Cu) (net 2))
 (segment (start 143.74 76.06) (end 143.74 75.96) (width 0.2) (layer B.Cu) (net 2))
 (segment (start 143.74 75.96) (end 144.9 74.8) (width 0.2) (layer B.Cu) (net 2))
 (segment (start 147.54 74.8) (end 148.82 73.52) (width 0.2) (layer B.Cu) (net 2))
 (segment (start 144.9 74.8) (end 147.54 74.8) (width 0.2) (layer B.Cu) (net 2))
 (segment (start 158.741314 80.06) (end 143.73 80.06) (width 1) (layer B.Cu) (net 2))
 (segment (start 161.52 77.281314) (end 158.741314 80.06) (width 1) (layer B.Cu) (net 2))
 (segment (start 161.52 76.06) (end 161.52 77.281314) (width 1) (layer B.Cu) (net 2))
 (segment (start 111.27 74) (end 111.14 73.87) (width 1) (layer F.Cu) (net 2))
 (segment (start 121.78 88.8) (end 121.91 88.8) (width 0.2) (layer B.Cu) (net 2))
 (segment (start 113.26 73.52) (end 115.8 73.52) (width 1) (layer B.Cu) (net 3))
 (segment (start 112.91 73.87) (end 113.26 73.52) (width 1) (layer B.Cu) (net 3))
 (segment (start 110.39929 79.3) (end 110.549999 79.450709) (width 0.2) (layer F.Cu) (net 12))
 (segment (start 111.200709 79.599949) (end 110.969991 79.830667) (width 0.2) (layer F.Cu) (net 12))
 (segment (start 117.56 85.87) (end 117.59 85.87) (width 1) (layer B.Cu) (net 11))
 (segment (start 117.56 88.57) (end 117.55 88.57) (width 1) (layer B.Cu) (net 4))
 (segment (start 117.56 88.67) (end 117.56 88.57) (width 0.2) (layer B.Cu) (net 4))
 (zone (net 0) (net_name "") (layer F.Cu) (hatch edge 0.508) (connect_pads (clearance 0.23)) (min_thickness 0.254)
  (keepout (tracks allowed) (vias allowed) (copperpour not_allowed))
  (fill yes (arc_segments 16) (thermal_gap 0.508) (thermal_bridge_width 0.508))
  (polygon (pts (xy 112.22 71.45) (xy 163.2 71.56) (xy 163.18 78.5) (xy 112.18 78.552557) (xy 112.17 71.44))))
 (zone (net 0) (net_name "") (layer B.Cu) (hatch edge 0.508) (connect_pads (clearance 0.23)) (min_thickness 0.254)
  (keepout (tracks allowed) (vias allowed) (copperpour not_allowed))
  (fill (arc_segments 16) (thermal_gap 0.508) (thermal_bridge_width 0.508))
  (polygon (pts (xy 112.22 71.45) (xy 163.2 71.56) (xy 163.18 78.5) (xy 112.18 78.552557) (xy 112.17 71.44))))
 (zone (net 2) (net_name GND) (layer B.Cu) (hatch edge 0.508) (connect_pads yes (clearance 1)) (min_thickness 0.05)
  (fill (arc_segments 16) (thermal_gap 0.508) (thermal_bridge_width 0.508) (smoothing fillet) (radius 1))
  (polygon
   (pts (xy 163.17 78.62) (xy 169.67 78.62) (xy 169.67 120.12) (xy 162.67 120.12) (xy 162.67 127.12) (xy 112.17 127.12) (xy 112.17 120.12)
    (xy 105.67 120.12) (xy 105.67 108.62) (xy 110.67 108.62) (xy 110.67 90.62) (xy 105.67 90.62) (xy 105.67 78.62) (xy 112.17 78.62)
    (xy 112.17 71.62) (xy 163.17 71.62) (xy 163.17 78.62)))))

